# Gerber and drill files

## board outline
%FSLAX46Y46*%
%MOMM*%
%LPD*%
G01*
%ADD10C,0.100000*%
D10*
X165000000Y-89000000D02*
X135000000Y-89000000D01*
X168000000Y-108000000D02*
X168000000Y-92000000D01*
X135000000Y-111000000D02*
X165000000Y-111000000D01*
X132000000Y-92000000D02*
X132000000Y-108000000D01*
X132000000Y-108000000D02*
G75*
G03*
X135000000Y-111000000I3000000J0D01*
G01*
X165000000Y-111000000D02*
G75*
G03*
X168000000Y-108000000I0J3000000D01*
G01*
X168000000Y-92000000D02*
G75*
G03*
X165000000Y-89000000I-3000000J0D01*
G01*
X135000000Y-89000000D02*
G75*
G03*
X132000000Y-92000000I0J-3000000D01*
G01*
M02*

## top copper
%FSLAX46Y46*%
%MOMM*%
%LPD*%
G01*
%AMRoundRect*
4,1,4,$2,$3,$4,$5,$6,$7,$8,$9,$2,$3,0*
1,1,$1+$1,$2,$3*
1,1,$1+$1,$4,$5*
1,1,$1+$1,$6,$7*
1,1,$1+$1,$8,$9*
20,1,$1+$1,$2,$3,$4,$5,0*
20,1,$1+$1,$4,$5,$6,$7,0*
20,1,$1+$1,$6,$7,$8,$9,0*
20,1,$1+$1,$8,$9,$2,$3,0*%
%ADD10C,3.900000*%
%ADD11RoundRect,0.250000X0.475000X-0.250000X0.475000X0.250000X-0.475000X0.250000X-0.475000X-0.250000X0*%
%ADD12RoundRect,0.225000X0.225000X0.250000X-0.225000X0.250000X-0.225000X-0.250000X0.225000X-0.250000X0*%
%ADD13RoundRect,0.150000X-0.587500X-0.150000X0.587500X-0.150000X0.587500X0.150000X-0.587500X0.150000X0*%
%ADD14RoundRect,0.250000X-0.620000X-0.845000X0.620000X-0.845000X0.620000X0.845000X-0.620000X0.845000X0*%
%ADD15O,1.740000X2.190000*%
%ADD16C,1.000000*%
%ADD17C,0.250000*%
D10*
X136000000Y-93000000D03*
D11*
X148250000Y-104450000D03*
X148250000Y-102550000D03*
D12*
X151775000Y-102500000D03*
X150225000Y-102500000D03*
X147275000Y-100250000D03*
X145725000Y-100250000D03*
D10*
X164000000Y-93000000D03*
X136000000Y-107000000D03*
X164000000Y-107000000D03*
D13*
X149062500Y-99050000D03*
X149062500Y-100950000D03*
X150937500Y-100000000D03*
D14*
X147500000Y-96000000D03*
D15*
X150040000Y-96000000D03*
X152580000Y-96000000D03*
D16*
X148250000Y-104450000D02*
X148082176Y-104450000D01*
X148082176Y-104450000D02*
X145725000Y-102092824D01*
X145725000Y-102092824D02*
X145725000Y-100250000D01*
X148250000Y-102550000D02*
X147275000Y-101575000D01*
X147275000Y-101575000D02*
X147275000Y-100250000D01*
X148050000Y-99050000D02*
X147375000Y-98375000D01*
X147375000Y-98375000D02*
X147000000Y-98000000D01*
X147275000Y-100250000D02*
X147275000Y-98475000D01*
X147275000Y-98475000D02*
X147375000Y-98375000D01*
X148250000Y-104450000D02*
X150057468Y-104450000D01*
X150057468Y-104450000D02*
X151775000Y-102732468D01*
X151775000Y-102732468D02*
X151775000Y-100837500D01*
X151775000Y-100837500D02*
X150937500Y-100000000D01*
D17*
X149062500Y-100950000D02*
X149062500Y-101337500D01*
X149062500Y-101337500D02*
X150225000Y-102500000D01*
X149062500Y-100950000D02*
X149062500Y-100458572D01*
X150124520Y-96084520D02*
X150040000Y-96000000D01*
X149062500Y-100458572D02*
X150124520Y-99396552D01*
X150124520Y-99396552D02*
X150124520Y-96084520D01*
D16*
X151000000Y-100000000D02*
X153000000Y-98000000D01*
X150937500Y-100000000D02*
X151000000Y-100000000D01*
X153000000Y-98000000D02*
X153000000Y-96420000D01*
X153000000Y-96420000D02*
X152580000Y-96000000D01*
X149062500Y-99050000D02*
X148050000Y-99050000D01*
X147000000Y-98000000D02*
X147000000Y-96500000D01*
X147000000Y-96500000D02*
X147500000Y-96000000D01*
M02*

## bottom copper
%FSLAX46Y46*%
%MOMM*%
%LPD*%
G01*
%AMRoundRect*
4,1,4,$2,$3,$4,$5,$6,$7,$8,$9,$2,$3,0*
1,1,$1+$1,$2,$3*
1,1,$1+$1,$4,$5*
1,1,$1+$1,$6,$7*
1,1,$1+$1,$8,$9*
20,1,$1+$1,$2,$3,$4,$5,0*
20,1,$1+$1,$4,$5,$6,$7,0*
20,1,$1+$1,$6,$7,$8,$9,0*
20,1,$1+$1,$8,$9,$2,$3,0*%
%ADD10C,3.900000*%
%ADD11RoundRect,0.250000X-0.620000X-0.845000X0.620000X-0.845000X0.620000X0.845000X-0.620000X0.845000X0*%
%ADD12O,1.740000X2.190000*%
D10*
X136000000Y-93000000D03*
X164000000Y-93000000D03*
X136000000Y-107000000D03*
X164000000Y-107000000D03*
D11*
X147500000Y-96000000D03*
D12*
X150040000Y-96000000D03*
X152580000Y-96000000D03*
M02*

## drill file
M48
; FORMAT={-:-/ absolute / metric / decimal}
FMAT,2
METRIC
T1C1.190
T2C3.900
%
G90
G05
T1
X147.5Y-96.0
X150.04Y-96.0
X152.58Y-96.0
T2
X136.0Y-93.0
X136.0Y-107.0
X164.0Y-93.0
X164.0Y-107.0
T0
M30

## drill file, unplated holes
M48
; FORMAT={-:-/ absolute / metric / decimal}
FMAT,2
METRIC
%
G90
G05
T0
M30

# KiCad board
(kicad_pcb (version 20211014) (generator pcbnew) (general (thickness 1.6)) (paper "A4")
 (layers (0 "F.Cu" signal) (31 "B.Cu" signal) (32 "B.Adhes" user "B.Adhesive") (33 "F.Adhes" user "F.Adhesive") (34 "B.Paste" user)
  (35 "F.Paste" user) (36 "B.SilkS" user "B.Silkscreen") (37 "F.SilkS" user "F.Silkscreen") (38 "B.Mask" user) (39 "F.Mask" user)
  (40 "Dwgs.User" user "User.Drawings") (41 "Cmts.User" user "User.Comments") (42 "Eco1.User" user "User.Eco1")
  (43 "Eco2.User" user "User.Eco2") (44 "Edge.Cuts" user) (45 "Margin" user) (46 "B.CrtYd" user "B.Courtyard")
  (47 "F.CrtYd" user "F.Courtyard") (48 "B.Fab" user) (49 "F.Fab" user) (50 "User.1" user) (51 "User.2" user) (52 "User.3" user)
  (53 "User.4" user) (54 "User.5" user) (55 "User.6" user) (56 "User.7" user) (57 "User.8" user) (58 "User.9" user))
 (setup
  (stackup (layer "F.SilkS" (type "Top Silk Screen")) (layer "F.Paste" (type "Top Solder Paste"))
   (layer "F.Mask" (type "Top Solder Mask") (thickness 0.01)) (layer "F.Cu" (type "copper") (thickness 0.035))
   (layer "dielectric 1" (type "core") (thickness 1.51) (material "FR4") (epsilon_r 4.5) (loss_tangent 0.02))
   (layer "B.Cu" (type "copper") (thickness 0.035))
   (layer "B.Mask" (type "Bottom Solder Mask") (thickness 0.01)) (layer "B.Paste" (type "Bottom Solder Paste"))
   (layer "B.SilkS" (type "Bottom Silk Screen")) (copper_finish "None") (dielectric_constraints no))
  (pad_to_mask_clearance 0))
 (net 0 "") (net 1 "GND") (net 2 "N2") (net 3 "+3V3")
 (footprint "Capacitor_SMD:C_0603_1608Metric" (layer "F.Cu") (at 151 102.5 180)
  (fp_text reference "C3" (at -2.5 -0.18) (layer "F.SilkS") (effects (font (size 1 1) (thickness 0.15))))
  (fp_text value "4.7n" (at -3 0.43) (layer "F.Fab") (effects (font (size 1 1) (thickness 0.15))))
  (pad "1" smd roundrect (at -0.775 0 180) (size 0.9 0.95) (layers "F.Cu" "F.Paste" "F.Mask") (roundrect_rratio 0.25) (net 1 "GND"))
  (pad "2" smd roundrect (at 0.775 0 180) (size 0.9 0.95) (layers "F.Cu" "F.Paste" "F.Mask") (roundrect_rratio 0.25) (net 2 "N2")))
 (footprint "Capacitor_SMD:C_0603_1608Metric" (layer "F.Cu") (at 146.5 100.25 180)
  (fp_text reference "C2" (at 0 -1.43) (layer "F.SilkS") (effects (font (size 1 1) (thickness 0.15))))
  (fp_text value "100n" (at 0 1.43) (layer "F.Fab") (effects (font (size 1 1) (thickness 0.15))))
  (pad "1" smd roundrect (at -0.775 0 180) (size 0.9 0.95) (layers "F.Cu" "F.Paste" "F.Mask") (roundrect_rratio 0.25) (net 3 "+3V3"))
  (pad "2" smd roundrect (at 0.775 0 180) (size 0.9 0.95) (layers "F.Cu" "F.Paste" "F.Mask") (roundrect_rratio 0.25) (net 1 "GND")))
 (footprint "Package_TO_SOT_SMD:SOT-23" (layer "F.Cu") (at 150 100)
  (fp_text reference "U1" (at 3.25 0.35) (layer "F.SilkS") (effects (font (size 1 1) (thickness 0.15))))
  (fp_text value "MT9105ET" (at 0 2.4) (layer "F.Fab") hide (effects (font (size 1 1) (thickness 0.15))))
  (pad "1" smd roundrect (at -0.9375 -0.95) (size 1.475 0.6) (layers "F.Cu" "F.Paste" "F.Mask") (roundrect_rratio 0.25) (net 3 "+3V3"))
  (pad "2" smd roundrect (at -0.9375 0.95) (size 1.475 0.6) (layers "F.Cu" "F.Paste" "F.Mask") (roundrect_rratio 0.25) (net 2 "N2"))
  (pad "3" smd roundrect (at 0.9375 0) (size 1.475 0.6) (layers "F.Cu" "F.Paste" "F.Mask") (roundrect_rratio 0.25) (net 1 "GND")))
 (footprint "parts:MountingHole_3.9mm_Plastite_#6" (layer "F.Cu") (at 164 93)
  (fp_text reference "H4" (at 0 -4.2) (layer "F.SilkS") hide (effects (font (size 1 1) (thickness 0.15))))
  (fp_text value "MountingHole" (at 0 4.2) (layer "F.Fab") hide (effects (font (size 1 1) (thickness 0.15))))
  (pad "" thru_hole circle (at 0 0) (size 3.9 3.9) (drill 3.9) (layers *.Cu *.Mask)))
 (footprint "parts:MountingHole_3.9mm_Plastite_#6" (layer "F.Cu") (at 136 93)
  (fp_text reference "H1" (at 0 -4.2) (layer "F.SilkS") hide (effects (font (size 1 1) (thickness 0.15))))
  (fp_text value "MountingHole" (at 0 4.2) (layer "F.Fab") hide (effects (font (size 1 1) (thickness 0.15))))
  (pad "" thru_hole circle (at 0 0) (size 3.9 3.9) (drill 3.9) (layers *.Cu *.Mask)))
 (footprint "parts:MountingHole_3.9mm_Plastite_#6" (layer "F.Cu") (at 164 107)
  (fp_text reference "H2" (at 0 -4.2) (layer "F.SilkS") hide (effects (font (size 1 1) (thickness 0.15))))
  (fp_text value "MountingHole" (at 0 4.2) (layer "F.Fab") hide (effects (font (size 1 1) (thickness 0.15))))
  (pad "" thru_hole circle (at 0 0) (size 3.9 3.9) (drill 3.9) (layers *.Cu *.Mask)))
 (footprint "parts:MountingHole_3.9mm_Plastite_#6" (layer "F.Cu") (at 136 107)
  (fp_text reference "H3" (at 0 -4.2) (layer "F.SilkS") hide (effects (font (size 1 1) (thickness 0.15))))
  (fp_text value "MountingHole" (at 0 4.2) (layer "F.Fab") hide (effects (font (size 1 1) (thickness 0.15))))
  (pad "" thru_hole circle (at 0 0) (size 3.9 3.9) (drill 3.9) (layers *.Cu *.Mask)))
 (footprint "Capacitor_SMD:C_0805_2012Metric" (layer "F.Cu") (at 148.25 103.5 90)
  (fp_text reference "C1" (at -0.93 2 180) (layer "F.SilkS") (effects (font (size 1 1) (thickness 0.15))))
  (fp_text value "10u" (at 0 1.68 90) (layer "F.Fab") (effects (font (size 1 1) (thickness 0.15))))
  (pad "1" smd roundrect (at -0.95 0 90) (size 1 1.45) (layers "F.Cu" "F.Paste" "F.Mask") (roundrect_rratio 0.25) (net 1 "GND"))
  (pad "2" smd roundrect (at 0.95 0 90) (size 1 1.45) (layers "F.Cu" "F.Paste" "F.Mask") (roundrect_rratio 0.25) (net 3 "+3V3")))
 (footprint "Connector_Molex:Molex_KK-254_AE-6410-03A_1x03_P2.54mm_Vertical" (layer "B.Cu") (at 147.5 96)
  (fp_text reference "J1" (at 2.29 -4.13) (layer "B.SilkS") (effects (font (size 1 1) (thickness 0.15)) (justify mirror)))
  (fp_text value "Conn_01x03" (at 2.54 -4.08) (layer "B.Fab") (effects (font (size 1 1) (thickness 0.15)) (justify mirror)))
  (pad "1" thru_hole roundrect (at 0 0) (size 1.74 2.19) (drill 1.19) (layers *.Cu *.Mask) (roundrect_rratio 0.1436781609) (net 3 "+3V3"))
  (pad "2" thru_hole oval (at 2.54 0) (size 1.74 2.19) (drill 1.19) (layers *.Cu *.Mask) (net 2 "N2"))
  (pad "3" thru_hole oval (at 5.08 0) (size 1.74 2.19) (drill 1.19) (layers *.Cu *.Mask) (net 1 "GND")))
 (gr_line (start 168 108) (end 168 92) (layer "Edge.Cuts") (width 0.1))
 (gr_arc (start 135 111) (mid 132.87868 110.12132) (end 132 108) (layer "Edge.Cuts") (width 0.1))
 (gr_arc (start 168 108) (mid 167.12132 110.12132) (end 165 111) (layer "Edge.Cuts") (width 0.1))
 (gr_arc (start 132 92) (mid 132.87868 89.87868) (end 135 89) (layer "Edge.Cuts") (width 0.1))
 (gr_arc (start 165 89) (mid 167.12132 89.87868) (end 168 92) (layer "Edge.Cuts") (width 0.1))
 (gr_line (start 132 92) (end 132 108) (layer "Edge.Cuts") (width 0.1))
 (gr_line (start 135 111) (end 165 111) (layer "Edge.Cuts") (width 0.1))
 (gr_line (start 165 89) (end 135 89) (layer "Edge.Cuts") (width 0.1))
 (segment (start 147.275 98.475) (end 147.375 98.375) (width 1) (layer "F.Cu") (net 3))
 (segment (start 149.0625 99.05) (end 148.05 99.05) (width 1) (layer "F.Cu") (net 3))
 (segment (start 147.375 98.375) (end 147 98) (width 1) (layer "F.Cu") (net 3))
 (segment (start 148.05 99.05) (end 147.375 98.375) (width 1) (layer "F.Cu") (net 3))
 (segment (start 147.275 100.25) (end 147.275 98.475) (width 1) (layer "F.Cu") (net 3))
 (segment (start 147 98) (end 147 96.5) (width 1) (layer "F.Cu") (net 3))
 (segment (start 147 96.5) (end 147.5 96) (width 1) (layer "F.Cu") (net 3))
 (segment (start 148.25 102.55) (end 147.275 101.575) (width 1) (layer "F.Cu") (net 3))
 (segment (start 147.275 101.575) (end 147.275 100.25) (width 1) (layer "F.Cu") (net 3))
 (segment (start 151.775 102.732468) (end 151.775 100.8375) (width 1) (layer "F.Cu") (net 1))
 (segment (start 148.25 104.45) (end 150.057468 104.45) (width 1) (layer "F.Cu") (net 1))
 (segment (start 145.725 102.092824) (end 145.725 100.25) (width 1) (layer "F.Cu") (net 1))
 (segment (start 150.9375 100) (end 151 100) (width 1) (layer "F.Cu") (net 1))
 (segment (start 151 100) (end 153 98) (width 1) (layer "F.Cu") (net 1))
 (segment (start 153 98) (end 153 96.42) (width 1) (layer "F.Cu") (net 1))
 (segment (start 151.775 100.8375) (end 150.9375 100) (width 1) (layer "F.Cu") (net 1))
 (segment (start 150.057468 104.45) (end 151.775 102.732468) (width 1) (layer "F.Cu") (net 1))
 (segment (start 153 96.42) (end 152.58 96) (width 1) (layer "F.Cu") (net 1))
 (segment (start 148.082176 104.45) (end 145.725 102.092824) (width 1) (layer "F.Cu") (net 1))
 (segment (start 148.25 104.45) (end 148.082176 104.45) (width 1) (layer "F.Cu") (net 1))
 (segment (start 150.12452 96.08452) (end 150.04 96) (width 0.25) (layer "F.Cu") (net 2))
 (segment (start 149.0625 100.95) (end 149.0625 100.458572) (width 0.25) (layer "F.Cu") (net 2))
 (segment (start 150.12452 99.396552) (end 150.12452 96.08452) (width 0.25) (layer "F.Cu") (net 2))
 (segment (start 149.0625 100.95) (end 149.0625 101.3375) (width 0.25) (layer "F.Cu") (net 2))
 (segment (start 149.0625 101.3375) (end 150.225 102.5) (width 0.25) (layer "F.Cu") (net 2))
 (segment (start 149.0625 100.458572) (end 150.12452 99.396552) (width 0.25) (layer "F.Cu") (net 2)))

